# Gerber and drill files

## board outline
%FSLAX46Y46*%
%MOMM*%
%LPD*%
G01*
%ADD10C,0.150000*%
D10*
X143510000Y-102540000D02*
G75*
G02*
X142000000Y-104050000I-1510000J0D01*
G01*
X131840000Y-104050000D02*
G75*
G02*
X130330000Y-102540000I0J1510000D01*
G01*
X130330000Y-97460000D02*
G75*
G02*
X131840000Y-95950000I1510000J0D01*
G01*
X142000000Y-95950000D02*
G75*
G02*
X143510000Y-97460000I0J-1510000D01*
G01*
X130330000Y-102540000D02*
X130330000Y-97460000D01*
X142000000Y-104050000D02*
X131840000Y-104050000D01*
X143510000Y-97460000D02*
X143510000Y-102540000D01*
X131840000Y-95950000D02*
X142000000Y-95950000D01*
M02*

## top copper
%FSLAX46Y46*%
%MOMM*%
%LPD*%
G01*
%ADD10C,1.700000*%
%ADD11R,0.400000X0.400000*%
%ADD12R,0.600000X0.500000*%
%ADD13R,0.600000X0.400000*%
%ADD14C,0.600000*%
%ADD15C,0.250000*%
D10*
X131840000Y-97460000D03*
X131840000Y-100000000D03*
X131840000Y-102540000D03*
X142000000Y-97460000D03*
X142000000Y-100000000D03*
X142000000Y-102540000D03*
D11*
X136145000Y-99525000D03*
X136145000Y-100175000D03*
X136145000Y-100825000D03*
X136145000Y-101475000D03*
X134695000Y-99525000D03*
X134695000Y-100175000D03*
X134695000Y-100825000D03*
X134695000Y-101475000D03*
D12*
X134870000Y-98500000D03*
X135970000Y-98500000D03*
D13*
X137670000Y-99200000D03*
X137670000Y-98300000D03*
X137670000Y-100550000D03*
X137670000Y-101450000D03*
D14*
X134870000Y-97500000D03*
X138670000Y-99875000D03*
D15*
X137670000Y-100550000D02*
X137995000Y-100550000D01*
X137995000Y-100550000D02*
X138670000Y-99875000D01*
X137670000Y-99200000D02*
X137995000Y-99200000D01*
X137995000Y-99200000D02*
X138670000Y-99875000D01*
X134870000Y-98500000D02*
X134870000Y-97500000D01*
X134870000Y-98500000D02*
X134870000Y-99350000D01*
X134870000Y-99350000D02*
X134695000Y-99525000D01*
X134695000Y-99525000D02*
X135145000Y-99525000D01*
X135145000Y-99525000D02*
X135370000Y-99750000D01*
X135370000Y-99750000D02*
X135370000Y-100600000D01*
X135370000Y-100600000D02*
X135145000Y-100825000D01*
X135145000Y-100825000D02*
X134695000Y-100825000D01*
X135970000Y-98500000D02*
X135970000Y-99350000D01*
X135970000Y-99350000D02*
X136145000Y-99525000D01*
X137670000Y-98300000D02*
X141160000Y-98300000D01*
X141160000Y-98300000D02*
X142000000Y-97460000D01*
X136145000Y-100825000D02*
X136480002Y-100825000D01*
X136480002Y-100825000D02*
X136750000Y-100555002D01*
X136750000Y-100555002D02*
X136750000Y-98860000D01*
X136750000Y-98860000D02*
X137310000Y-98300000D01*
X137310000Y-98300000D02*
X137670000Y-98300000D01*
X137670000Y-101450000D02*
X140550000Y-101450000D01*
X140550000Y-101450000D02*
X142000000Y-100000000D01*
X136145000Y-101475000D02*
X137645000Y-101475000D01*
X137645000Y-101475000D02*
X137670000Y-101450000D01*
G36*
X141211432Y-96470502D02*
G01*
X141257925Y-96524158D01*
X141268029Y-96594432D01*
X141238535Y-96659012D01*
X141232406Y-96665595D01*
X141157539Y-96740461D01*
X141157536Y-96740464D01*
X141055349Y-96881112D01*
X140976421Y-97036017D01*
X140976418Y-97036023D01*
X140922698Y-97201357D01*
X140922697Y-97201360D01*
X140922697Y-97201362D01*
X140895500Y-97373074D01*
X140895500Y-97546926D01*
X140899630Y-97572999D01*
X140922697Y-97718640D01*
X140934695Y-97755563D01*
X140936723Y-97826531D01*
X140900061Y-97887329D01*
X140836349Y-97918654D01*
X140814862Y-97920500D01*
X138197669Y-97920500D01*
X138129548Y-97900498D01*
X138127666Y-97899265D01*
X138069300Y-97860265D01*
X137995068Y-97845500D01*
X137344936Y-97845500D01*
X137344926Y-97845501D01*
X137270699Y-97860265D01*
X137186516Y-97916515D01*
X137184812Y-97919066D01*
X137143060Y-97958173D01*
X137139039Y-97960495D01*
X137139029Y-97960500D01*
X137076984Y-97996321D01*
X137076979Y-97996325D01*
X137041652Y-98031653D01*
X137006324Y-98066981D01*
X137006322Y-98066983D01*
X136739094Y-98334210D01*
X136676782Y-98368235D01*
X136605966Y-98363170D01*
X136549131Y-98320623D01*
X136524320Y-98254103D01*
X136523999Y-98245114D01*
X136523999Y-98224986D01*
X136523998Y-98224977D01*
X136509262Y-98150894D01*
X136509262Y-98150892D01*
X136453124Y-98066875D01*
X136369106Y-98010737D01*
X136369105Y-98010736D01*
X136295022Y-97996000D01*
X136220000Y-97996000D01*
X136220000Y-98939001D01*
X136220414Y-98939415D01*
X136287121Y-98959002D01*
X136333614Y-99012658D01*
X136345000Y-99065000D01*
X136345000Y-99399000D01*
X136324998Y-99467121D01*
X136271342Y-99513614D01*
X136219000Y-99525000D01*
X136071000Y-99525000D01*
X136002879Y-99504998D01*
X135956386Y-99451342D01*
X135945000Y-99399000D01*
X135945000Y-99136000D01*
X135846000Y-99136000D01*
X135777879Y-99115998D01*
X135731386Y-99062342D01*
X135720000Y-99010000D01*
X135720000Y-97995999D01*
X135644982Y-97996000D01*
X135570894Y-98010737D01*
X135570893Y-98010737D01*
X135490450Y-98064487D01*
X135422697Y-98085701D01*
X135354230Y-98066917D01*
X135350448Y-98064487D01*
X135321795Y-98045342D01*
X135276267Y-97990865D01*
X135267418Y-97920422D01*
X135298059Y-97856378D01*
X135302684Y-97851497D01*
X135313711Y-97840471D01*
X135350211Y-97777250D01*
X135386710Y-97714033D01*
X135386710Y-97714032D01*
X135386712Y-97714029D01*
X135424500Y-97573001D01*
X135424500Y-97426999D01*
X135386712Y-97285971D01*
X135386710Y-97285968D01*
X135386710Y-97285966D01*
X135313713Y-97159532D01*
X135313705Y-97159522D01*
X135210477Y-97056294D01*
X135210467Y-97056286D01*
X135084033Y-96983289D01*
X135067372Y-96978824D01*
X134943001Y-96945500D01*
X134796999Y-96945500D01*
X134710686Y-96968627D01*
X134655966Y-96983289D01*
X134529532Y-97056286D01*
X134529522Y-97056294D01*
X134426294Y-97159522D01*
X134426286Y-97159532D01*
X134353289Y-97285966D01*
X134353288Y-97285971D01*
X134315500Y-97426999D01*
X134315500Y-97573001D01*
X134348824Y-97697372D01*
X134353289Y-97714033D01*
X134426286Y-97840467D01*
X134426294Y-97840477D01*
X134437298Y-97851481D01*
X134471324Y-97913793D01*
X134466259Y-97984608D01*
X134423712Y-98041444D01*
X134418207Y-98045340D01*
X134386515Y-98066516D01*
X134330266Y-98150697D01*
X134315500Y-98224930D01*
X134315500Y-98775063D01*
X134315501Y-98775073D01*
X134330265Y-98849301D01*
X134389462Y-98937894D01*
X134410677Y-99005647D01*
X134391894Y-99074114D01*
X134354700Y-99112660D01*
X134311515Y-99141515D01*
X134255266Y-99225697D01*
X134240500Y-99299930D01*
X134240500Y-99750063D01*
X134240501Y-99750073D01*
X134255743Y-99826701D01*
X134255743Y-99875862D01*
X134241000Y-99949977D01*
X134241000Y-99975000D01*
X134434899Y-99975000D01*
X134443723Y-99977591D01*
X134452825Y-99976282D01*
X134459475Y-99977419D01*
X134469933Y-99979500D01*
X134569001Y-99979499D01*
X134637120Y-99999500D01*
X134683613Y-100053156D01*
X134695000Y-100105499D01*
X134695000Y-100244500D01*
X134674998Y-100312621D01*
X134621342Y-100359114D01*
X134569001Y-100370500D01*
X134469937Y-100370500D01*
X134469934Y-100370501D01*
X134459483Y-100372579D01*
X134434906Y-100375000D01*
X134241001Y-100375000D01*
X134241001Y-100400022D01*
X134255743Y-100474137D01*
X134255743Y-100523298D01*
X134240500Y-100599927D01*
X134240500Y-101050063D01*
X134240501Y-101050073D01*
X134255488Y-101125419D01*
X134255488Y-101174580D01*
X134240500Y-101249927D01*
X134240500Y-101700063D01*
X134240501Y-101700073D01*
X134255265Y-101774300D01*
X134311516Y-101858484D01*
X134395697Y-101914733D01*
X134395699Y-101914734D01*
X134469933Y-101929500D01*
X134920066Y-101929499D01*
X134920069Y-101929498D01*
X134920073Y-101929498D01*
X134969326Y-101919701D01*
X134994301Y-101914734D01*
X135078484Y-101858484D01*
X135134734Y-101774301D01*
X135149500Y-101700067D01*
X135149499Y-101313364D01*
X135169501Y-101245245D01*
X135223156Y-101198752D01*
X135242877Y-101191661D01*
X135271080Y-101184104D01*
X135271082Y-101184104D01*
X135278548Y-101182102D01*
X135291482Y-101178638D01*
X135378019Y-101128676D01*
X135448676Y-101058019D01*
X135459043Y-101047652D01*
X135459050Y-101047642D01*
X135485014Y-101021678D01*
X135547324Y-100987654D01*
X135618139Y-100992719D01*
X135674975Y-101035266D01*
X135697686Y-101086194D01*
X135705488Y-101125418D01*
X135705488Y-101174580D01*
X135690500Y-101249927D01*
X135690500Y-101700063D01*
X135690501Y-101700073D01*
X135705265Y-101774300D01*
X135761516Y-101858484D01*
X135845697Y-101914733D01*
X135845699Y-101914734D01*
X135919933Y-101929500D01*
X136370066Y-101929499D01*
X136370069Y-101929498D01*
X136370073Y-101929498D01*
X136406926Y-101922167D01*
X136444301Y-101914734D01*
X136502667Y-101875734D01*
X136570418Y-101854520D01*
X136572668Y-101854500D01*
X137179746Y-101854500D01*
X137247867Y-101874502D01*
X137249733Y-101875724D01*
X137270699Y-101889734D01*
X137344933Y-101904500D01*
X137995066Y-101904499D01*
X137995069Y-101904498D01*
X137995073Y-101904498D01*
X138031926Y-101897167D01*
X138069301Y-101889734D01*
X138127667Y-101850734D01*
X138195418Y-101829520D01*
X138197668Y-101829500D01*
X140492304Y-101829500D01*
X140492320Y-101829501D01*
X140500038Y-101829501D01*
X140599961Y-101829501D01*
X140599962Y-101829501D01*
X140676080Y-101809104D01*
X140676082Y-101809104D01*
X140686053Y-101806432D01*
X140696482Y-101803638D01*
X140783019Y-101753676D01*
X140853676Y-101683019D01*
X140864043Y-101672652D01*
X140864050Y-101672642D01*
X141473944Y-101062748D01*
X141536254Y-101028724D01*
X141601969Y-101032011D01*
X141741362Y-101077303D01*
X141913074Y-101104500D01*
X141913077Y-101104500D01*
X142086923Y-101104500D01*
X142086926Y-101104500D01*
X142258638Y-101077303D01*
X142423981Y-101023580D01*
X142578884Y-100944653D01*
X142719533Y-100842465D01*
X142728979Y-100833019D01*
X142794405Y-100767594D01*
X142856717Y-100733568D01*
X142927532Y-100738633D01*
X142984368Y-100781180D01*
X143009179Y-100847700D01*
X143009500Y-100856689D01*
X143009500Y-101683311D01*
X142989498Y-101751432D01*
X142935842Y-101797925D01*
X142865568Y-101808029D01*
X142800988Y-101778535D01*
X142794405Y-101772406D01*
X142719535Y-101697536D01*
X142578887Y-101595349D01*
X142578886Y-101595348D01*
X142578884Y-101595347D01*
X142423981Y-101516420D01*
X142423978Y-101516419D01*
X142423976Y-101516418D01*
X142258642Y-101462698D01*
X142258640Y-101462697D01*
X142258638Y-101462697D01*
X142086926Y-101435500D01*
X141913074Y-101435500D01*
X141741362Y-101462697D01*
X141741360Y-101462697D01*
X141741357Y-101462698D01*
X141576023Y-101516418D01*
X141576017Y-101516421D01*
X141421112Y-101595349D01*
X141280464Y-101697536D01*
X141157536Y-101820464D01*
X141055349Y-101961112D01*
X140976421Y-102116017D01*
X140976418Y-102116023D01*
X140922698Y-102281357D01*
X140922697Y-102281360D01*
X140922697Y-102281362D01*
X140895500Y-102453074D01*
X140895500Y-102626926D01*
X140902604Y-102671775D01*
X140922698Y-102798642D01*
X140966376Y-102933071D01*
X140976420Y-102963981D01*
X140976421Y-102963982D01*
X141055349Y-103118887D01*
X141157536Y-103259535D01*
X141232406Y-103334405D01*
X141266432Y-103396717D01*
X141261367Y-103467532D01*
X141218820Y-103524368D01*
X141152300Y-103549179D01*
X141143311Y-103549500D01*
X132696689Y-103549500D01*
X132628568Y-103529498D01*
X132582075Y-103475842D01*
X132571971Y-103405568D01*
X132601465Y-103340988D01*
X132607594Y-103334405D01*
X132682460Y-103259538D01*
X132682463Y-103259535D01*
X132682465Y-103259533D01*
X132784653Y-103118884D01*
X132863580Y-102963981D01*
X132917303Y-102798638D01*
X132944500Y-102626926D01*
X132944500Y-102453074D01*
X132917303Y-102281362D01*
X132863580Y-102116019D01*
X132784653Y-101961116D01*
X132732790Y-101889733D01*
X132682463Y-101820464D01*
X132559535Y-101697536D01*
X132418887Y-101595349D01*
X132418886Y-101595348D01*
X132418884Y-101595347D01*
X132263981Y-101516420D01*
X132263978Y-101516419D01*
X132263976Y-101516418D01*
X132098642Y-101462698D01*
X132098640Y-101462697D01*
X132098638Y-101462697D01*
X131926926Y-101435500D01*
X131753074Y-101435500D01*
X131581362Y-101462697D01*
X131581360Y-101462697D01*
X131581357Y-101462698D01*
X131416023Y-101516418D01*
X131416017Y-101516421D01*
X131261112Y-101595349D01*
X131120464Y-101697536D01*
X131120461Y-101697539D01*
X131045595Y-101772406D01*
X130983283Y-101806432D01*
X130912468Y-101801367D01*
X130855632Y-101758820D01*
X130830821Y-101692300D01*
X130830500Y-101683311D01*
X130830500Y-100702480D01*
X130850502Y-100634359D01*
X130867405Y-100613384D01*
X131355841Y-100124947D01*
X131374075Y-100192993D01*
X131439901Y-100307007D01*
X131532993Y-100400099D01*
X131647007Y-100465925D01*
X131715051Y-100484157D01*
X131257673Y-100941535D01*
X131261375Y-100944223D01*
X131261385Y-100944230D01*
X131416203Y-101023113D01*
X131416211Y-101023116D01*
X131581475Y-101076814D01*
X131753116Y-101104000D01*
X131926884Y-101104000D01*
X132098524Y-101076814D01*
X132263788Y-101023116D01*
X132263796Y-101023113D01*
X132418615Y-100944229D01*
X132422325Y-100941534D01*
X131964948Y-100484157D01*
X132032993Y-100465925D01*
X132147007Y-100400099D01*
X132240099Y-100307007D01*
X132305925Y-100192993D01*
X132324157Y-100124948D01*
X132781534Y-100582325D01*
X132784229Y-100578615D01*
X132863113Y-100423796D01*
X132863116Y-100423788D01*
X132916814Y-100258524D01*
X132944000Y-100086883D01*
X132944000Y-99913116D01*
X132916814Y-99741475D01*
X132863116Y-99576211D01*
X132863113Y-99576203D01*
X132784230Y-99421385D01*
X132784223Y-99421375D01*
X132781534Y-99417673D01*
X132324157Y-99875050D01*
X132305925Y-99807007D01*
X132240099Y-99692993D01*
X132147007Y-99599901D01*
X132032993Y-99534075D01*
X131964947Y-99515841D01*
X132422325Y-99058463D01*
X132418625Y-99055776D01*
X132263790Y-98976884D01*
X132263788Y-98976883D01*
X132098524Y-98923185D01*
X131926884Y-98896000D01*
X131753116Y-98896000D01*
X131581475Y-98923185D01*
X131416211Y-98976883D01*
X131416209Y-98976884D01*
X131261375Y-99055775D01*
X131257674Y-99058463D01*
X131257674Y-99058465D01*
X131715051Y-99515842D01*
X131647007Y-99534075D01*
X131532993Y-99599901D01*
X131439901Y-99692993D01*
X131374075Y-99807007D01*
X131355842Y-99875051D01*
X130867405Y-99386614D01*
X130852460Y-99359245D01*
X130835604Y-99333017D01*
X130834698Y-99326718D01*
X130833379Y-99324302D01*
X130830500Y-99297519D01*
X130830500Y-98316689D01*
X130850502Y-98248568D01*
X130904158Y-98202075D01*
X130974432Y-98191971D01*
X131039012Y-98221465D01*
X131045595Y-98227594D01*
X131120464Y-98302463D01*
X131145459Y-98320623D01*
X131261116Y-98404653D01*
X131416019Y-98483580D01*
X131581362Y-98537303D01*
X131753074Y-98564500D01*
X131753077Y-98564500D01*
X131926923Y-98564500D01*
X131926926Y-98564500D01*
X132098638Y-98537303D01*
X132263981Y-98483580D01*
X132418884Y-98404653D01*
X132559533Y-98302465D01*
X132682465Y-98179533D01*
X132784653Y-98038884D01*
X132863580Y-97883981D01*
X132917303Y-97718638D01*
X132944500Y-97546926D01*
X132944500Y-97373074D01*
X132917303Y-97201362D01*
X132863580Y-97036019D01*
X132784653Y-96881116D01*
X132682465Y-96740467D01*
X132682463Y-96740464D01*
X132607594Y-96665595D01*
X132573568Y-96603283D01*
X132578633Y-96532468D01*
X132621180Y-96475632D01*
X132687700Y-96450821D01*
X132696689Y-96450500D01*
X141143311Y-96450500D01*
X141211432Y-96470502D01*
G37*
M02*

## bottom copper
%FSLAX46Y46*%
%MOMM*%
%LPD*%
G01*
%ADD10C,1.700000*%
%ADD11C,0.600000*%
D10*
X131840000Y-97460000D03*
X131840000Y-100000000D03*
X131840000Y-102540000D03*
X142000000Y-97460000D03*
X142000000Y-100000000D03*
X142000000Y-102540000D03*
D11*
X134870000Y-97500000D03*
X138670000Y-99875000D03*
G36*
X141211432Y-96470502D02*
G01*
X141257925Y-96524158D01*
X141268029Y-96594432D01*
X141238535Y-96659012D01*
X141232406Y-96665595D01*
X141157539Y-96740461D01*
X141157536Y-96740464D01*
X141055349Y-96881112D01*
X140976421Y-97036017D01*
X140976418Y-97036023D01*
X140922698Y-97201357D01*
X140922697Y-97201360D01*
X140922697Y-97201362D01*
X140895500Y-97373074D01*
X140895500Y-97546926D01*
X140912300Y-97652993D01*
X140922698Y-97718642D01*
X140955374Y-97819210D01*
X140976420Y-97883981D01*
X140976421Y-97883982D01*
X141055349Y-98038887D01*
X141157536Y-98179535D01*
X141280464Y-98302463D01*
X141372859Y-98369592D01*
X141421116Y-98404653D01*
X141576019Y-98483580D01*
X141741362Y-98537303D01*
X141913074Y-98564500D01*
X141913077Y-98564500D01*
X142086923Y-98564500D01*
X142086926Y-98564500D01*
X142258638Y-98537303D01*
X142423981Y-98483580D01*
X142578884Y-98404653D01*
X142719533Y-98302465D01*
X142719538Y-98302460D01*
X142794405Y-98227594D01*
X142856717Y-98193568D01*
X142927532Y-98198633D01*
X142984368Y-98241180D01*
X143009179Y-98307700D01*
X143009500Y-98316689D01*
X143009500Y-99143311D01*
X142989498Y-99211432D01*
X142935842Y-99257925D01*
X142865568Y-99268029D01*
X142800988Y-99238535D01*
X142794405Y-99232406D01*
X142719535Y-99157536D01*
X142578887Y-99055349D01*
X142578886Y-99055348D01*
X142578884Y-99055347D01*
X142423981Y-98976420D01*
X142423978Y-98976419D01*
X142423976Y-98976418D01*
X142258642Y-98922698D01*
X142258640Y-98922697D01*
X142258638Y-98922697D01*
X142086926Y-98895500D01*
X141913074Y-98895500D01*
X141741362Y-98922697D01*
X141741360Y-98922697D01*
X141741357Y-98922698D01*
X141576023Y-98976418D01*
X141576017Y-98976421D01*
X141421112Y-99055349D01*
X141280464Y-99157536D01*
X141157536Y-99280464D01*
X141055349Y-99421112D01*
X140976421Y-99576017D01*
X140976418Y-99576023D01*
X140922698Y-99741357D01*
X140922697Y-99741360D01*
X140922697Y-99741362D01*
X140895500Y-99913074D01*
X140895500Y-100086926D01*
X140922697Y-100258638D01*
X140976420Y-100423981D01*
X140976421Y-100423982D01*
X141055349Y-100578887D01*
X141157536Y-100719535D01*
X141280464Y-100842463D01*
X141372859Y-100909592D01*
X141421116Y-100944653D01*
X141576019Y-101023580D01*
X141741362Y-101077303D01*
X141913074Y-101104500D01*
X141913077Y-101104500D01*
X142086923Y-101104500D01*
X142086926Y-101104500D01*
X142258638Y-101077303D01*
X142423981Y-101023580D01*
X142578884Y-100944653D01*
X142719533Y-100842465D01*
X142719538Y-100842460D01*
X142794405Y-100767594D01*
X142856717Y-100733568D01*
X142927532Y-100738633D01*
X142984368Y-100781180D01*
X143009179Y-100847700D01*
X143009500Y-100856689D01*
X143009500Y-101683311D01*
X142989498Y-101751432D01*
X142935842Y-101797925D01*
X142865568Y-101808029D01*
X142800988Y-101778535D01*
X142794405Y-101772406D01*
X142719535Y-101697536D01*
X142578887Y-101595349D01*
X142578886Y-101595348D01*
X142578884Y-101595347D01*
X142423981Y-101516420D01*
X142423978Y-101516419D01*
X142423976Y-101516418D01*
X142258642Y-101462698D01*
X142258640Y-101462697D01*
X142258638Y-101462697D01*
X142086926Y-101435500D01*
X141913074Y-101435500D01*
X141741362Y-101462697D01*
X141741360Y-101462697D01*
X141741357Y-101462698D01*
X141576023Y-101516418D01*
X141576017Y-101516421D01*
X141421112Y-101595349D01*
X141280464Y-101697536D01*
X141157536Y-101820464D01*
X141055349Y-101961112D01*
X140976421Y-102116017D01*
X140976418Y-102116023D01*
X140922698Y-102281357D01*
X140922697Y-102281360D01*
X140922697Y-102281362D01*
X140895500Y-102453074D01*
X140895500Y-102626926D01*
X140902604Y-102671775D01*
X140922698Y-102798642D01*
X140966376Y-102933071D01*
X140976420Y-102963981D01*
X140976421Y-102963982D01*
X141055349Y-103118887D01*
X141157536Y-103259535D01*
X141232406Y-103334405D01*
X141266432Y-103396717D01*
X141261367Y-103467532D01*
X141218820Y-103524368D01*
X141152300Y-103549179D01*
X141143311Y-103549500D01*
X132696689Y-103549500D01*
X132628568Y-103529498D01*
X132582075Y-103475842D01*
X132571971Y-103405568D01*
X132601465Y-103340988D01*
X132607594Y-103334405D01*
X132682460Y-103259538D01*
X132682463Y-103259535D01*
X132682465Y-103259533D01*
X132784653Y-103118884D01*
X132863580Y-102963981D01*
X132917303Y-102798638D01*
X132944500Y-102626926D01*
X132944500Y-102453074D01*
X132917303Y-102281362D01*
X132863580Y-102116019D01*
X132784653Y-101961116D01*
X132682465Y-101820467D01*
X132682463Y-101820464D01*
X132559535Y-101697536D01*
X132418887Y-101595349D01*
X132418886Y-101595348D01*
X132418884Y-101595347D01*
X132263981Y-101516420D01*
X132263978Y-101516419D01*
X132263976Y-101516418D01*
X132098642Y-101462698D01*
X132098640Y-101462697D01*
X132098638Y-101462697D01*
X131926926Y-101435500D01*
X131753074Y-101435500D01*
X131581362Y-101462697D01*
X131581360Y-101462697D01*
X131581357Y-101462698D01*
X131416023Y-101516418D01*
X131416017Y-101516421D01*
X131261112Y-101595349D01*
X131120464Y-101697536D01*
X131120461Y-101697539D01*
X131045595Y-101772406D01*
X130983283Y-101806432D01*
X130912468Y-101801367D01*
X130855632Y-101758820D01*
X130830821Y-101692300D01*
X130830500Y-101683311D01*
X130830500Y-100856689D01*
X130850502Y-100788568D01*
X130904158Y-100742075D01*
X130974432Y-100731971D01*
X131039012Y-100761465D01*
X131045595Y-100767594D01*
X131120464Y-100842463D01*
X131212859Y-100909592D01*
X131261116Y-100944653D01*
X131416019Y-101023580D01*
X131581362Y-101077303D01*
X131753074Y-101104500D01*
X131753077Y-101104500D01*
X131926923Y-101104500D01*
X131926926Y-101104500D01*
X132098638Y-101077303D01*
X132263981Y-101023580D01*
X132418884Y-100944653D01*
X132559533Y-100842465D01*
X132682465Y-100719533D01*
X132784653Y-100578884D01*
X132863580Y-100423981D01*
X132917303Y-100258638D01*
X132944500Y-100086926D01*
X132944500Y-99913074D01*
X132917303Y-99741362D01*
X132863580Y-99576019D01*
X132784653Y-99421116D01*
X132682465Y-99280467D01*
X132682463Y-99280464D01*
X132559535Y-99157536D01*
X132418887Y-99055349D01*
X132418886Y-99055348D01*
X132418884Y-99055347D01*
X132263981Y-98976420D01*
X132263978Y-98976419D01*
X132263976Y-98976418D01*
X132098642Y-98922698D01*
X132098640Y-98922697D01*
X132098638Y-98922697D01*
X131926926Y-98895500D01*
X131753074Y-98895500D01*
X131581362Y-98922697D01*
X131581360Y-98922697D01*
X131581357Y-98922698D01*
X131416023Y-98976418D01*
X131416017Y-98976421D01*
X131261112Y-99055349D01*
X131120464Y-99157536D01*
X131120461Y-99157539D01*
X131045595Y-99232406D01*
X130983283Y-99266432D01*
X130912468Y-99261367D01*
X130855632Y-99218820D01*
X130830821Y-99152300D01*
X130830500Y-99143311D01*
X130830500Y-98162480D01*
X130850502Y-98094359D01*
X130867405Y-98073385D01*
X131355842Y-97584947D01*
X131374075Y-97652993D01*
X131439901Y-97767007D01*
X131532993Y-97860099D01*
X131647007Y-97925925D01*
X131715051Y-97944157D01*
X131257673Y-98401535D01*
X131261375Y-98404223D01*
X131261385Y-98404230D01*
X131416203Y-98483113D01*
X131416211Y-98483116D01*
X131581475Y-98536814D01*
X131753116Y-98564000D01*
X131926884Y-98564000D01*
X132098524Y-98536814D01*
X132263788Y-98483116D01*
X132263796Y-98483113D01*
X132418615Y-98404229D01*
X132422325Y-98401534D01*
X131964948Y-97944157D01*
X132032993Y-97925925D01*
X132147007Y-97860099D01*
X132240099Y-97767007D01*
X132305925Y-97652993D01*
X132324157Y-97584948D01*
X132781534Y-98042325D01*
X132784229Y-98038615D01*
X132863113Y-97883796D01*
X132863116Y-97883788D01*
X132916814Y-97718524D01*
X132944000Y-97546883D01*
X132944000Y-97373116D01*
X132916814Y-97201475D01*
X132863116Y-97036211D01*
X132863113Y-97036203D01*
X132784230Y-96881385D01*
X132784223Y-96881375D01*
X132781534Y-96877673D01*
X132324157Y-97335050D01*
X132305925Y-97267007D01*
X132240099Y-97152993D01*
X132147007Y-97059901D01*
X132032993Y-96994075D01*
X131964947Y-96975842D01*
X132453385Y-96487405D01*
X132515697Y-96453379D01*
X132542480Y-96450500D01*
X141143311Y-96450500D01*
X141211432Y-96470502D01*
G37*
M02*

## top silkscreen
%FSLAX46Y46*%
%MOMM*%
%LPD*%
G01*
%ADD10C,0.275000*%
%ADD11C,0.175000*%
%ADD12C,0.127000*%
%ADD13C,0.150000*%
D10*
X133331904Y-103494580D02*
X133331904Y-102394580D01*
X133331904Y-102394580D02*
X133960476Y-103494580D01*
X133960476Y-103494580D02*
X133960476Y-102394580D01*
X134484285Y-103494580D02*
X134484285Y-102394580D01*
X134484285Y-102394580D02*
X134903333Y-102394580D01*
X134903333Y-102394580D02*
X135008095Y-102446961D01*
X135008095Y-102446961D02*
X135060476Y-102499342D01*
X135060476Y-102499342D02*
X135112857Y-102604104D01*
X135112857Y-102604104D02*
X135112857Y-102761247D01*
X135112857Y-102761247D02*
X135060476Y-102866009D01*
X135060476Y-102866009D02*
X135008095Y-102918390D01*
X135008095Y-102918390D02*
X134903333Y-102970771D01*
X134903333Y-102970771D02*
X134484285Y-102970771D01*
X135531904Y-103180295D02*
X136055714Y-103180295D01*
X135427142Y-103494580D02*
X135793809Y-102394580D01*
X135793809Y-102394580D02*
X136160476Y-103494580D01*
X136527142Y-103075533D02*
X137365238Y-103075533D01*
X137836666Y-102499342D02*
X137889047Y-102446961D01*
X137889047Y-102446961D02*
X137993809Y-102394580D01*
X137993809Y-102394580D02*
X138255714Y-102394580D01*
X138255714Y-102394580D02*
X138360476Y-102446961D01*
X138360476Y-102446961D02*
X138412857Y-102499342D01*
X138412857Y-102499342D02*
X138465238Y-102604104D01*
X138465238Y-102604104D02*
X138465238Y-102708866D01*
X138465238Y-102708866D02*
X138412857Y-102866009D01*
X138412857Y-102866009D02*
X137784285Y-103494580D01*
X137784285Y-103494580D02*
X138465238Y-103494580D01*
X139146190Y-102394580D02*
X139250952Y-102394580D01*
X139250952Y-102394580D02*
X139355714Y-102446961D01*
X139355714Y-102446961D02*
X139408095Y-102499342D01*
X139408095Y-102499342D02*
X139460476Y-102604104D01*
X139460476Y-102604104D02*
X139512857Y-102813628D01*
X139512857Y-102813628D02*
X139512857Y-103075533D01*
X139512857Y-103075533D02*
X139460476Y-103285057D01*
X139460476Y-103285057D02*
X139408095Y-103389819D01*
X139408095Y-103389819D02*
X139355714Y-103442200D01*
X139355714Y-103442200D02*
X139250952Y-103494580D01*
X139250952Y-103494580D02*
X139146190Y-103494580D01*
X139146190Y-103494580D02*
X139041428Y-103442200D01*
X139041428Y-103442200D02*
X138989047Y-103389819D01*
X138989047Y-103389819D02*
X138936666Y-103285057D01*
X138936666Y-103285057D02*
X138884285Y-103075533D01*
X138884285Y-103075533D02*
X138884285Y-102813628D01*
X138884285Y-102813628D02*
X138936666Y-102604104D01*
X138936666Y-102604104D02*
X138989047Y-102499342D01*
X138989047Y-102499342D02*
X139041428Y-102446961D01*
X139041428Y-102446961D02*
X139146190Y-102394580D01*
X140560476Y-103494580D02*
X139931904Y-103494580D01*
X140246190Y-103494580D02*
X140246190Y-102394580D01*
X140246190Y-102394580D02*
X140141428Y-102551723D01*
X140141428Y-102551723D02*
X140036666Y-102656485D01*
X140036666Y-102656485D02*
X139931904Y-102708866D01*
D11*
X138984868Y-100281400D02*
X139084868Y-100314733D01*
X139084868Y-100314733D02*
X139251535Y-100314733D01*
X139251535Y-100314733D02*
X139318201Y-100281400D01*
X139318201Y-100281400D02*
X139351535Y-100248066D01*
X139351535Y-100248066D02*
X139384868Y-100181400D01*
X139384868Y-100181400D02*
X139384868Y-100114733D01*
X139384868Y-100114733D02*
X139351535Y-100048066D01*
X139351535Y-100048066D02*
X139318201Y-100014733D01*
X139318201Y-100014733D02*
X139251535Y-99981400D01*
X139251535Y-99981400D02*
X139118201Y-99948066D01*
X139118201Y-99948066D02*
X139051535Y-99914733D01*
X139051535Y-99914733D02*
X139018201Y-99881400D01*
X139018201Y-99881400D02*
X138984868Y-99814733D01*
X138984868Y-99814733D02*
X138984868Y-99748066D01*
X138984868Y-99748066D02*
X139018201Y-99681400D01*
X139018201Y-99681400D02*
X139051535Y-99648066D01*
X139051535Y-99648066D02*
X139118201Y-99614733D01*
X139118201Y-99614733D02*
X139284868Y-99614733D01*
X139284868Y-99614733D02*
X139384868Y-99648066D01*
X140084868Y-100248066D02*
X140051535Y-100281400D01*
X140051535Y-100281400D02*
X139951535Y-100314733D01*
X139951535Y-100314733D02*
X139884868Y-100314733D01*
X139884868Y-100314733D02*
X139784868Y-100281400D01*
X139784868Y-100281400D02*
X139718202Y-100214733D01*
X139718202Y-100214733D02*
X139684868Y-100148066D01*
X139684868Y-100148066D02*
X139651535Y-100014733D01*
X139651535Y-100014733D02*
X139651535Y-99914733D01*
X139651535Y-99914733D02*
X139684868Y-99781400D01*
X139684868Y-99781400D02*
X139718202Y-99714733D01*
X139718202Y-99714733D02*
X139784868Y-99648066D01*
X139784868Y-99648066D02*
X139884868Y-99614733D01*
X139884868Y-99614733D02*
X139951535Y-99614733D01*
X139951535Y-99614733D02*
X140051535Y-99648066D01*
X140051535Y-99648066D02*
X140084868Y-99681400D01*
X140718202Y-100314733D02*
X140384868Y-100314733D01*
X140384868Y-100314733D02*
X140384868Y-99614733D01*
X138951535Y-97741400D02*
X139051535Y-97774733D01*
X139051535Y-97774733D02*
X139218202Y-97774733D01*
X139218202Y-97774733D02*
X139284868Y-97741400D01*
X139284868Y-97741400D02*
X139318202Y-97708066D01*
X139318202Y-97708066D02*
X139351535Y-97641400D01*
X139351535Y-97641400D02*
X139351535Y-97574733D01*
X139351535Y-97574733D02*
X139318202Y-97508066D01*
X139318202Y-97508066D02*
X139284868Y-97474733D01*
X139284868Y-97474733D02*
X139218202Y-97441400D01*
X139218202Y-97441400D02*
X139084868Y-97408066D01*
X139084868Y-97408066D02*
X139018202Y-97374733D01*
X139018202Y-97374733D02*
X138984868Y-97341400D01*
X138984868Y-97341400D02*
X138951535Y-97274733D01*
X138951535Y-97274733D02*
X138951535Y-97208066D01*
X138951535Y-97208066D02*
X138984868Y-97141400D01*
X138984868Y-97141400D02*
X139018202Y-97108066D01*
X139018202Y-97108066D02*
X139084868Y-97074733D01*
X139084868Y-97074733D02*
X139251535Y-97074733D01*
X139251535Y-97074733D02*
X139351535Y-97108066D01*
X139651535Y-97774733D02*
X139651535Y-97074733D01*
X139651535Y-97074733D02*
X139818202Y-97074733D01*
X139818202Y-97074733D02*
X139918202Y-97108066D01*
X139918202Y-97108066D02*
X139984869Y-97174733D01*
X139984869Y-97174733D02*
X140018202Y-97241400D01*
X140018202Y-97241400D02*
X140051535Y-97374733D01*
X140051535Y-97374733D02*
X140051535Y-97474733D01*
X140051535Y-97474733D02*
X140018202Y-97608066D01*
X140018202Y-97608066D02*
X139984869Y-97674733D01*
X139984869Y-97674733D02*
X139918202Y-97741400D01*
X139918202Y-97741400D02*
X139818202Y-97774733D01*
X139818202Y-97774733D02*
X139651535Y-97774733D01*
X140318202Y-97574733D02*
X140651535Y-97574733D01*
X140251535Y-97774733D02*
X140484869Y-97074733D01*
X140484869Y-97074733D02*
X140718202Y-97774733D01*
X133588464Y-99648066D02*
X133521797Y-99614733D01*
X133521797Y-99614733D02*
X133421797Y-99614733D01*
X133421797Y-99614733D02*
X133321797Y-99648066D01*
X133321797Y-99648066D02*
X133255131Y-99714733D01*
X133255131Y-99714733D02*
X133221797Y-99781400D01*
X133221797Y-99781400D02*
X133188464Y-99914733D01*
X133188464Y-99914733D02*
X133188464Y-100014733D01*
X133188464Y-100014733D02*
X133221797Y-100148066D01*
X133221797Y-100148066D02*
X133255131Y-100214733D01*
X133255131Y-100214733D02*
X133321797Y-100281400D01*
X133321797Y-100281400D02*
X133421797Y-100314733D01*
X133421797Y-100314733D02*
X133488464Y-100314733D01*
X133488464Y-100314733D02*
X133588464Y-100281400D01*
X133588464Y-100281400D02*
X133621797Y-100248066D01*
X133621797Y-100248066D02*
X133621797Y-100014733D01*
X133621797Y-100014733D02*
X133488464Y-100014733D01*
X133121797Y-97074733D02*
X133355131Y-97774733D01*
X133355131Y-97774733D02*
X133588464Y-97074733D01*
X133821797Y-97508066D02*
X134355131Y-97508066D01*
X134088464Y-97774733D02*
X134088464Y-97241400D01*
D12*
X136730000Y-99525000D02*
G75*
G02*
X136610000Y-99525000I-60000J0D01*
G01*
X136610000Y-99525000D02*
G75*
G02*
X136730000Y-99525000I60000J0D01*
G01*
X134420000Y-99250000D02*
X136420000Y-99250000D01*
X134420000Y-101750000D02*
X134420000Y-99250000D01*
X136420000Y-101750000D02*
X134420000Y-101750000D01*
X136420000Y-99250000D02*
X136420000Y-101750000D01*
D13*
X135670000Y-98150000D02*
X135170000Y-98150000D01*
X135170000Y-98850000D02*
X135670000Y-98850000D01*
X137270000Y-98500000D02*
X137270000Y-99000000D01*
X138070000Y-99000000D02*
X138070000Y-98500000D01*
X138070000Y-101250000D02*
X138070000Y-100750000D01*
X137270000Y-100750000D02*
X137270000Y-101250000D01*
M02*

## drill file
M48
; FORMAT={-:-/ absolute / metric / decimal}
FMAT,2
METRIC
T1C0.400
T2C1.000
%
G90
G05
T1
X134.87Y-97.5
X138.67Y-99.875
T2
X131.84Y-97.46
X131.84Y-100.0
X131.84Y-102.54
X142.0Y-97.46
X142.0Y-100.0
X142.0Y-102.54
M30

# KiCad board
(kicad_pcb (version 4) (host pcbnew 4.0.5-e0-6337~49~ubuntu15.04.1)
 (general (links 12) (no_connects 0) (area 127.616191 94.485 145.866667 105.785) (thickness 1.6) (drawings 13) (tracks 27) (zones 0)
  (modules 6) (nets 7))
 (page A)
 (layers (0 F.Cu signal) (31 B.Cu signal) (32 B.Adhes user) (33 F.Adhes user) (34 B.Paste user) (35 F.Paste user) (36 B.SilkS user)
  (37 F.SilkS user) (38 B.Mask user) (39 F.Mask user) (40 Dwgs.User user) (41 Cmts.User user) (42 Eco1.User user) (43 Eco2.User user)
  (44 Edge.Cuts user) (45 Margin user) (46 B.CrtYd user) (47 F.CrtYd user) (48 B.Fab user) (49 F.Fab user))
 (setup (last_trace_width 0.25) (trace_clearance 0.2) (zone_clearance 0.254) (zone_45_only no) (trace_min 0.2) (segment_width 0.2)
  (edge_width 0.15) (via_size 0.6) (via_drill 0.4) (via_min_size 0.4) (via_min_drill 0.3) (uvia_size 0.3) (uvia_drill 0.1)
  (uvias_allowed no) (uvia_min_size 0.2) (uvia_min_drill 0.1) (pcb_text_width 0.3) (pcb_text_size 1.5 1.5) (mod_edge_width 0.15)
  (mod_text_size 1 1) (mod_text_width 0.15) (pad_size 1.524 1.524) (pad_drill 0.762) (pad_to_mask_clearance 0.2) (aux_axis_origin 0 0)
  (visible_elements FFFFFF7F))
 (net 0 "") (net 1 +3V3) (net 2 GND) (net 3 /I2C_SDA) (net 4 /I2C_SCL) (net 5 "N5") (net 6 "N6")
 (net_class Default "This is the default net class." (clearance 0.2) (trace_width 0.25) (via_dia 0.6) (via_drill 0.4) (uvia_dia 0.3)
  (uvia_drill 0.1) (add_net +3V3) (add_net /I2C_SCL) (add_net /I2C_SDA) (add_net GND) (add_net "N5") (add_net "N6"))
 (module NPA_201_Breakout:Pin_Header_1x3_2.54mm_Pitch (layer F.Cu) (at 131.84 97.46)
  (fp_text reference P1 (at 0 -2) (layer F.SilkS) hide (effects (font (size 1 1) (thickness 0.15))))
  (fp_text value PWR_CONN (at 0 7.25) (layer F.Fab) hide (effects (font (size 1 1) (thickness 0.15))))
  (pad 1 thru_hole circle (at 0 0) (size 1.7 1.7) (drill 1) (layers *.Cu *.Mask) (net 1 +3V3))
  (pad 2 thru_hole circle (at 0 2.54) (size 1.7 1.7) (drill 1) (layers *.Cu *.Mask) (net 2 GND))
  (pad 3 thru_hole circle (at 0 5.08) (size 1.7 1.7) (drill 1) (layers *.Cu *.Mask)))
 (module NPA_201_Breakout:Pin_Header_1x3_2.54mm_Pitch (layer F.Cu) (at 142 97.46)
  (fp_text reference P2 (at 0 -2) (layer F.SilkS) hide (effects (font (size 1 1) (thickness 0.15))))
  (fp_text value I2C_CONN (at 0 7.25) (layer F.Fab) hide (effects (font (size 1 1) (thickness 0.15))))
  (pad 1 thru_hole circle (at 0 0) (size 1.7 1.7) (drill 1) (layers *.Cu *.Mask) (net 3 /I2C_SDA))
  (pad 2 thru_hole circle (at 0 2.54) (size 1.7 1.7) (drill 1) (layers *.Cu *.Mask) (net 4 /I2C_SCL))
  (pad 3 thru_hole circle (at 0 5.08) (size 1.7 1.7) (drill 1) (layers *.Cu *.Mask)))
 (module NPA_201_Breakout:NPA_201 (layer F.Cu) (at 135.42 100.5 270)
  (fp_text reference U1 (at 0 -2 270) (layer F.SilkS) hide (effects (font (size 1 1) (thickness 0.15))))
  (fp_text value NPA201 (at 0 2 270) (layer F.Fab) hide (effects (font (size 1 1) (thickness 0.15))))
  (fp_circle (center -0.975 -1.25) (end -0.975 -1.19) (layer F.SilkS) (width 0.127))
  (fp_line (start -1.25 1) (end -1.25 -1) (layer F.SilkS) (width 0.127))
  (fp_line (start 1.25 1) (end -1.25 1) (layer F.SilkS) (width 0.127))
  (fp_line (start 1.25 -1) (end 1.25 1) (layer F.SilkS) (width 0.127))
  (fp_line (start -1.25 -1) (end 1.25 -1) (layer F.SilkS) (width 0.127))
  (pad 1 smd rect (at -0.975 -0.725 270) (size 0.4 0.4) (layers F.Cu F.Paste F.Mask) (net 2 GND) (solder_mask_margin 0.05)
   (solder_paste_margin -0.025))
  (pad 2 smd rect (at -0.325 -0.725 270) (size 0.4 0.4) (layers F.Cu F.Paste F.Mask) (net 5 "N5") (solder_mask_margin 0.05)
   (solder_paste_margin -0.025))
  (pad 3 smd rect (at 0.325 -0.725 270) (size 0.4 0.4) (layers F.Cu F.Paste F.Mask) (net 3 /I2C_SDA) (solder_mask_margin 0.05)
   (solder_paste_margin -0.025))
  (pad 4 smd rect (at 0.975 -0.725 270) (size 0.4 0.4) (layers F.Cu F.Paste F.Mask) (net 4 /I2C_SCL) (solder_mask_margin 0.05)
   (solder_paste_margin -0.025))
  (pad 8 smd rect (at -0.975 0.725 270) (size 0.4 0.4) (layers F.Cu F.Paste F.Mask) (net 1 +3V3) (solder_mask_margin 0.05)
   (solder_paste_margin -0.025))
  (pad 7 smd rect (at -0.325 0.725 270) (size 0.4 0.4) (layers F.Cu F.Paste F.Mask) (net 2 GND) (solder_mask_margin 0.05)
   (solder_paste_margin -0.025))
  (pad 6 smd rect (at 0.325 0.725 270) (size 0.4 0.4) (layers F.Cu F.Paste F.Mask) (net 1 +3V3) (solder_mask_margin 0.05)
   (solder_paste_margin -0.025))
  (pad 5 smd rect (at 0.975 0.725 270) (size 0.4 0.4) (layers F.Cu F.Paste F.Mask) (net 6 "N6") (solder_mask_margin 0.05)
   (solder_paste_margin -0.025)))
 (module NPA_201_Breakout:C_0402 (layer F.Cu) (at 135.42 98.5)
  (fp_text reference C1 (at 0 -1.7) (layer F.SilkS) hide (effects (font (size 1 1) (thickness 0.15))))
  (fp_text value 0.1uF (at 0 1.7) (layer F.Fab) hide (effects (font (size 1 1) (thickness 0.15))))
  (fp_line (start 0.25 -0.35) (end -0.25 -0.35) (layer F.SilkS) (width 0.15))
  (fp_line (start -0.25 0.35) (end 0.25 0.35) (layer F.SilkS) (width 0.15))
  (pad 1 smd rect (at -0.55 0) (size 0.6 0.5) (layers F.Cu F.Paste F.Mask) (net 1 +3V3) (solder_mask_margin 0.1))
  (pad 2 smd rect (at 0.55 0) (size 0.6 0.5) (layers F.Cu F.Paste F.Mask) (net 2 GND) (solder_mask_margin 0.1)))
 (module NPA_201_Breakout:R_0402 (layer F.Cu) (at 137.67 98.75 90)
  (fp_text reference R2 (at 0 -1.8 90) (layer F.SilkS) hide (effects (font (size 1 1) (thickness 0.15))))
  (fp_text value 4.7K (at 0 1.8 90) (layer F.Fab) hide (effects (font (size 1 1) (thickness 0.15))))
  (fp_line (start 0.25 -0.4) (end -0.25 -0.4) (layer F.SilkS) (width 0.15))
  (fp_line (start -0.25 0.4) (end 0.25 0.4) (layer F.SilkS) (width 0.15))
  (pad 1 smd rect (at -0.45 0 90) (size 0.4 0.6) (layers F.Cu F.Paste F.Mask) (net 1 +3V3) (solder_mask_margin 0.1))
  (pad 2 smd rect (at 0.45 0 90) (size 0.4 0.6) (layers F.Cu F.Paste F.Mask) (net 3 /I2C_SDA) (solder_mask_margin 0.1)))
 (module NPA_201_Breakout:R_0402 (layer F.Cu) (at 137.67 101 270)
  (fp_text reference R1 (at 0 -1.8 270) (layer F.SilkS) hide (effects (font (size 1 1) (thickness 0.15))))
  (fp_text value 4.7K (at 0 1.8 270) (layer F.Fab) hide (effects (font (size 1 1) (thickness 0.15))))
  (fp_line (start 0.25 -0.4) (end -0.25 -0.4) (layer F.SilkS) (width 0.15))
  (fp_line (start -0.25 0.4) (end 0.25 0.4) (layer F.SilkS) (width 0.15))
  (pad 1 smd rect (at -0.45 0 270) (size 0.4 0.6) (layers F.Cu F.Paste F.Mask) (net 1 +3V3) (solder_mask_margin 0.1))
  (pad 2 smd rect (at 0.45 0 270) (size 0.4 0.6) (layers F.Cu F.Paste F.Mask) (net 4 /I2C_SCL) (solder_mask_margin 0.1)))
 (gr_arc (start 142 102.54) (end 143.51 102.54) (angle 90) (layer Edge.Cuts) (width 0.15))
 (gr_arc (start 131.84 102.54) (end 131.84 104.05) (angle 90) (layer Edge.Cuts) (width 0.15))
 (gr_arc (start 131.84 97.46) (end 130.33 97.46) (angle 90) (layer Edge.Cuts) (width 0.15))
 (gr_arc (start 142 97.46) (end 142 95.95) (angle 90) (layer Edge.Cuts) (width 0.15))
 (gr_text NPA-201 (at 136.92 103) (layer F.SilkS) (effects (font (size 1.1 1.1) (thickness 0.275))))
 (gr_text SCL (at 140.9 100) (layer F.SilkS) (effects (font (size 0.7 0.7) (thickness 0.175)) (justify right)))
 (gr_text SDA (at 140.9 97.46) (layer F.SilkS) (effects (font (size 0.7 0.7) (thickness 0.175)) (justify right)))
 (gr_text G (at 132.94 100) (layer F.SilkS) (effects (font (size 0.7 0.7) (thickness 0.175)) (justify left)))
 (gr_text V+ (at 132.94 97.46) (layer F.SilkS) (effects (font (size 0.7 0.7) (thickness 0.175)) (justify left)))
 (gr_line (start 130.33 102.54) (end 130.33 97.46) (layer Edge.Cuts) (width 0.15))
 (gr_line (start 142 104.05) (end 131.84 104.05) (layer Edge.Cuts) (width 0.15))
 (gr_line (start 143.51 97.46) (end 143.51 102.54) (layer Edge.Cuts) (width 0.15))
 (gr_line (start 131.84 95.95) (end 142 95.95) (layer Edge.Cuts) (width 0.15))
 (segment (start 137.67 100.55) (end 137.995 100.55) (width 0.25) (layer F.Cu) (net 1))
 (segment (start 137.995 100.55) (end 138.67 99.875) (width 0.25) (layer F.Cu) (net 1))
 (segment (start 137.67 99.2) (end 137.995 99.2) (width 0.25) (layer F.Cu) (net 1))
 (segment (start 137.995 99.2) (end 138.67 99.875) (width 0.25) (layer F.Cu) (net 1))
 (segment (start 134.87 98.5) (end 134.87 97.5) (width 0.25) (layer F.Cu) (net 1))
 (via (at 134.87 97.5) (size 0.6) (drill 0.4) (layers F.Cu B.Cu) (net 1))
 (via (at 138.67 99.875) (size 0.6) (drill 0.4) (layers F.Cu B.Cu) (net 1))
 (segment (start 134.87 98.5) (end 134.87 99.35) (width 0.25) (layer F.Cu) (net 1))
 (segment (start 134.87 99.35) (end 134.695 99.525) (width 0.25) (layer F.Cu) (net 1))
 (segment (start 134.695 99.525) (end 135.145 99.525) (width 0.25) (layer F.Cu) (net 1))
 (segment (start 135.145 99.525) (end 135.37 99.75) (width 0.25) (layer F.Cu) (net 1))
 (segment (start 135.37 99.75) (end 135.37 100.6) (width 0.25) (layer F.Cu) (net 1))
 (segment (start 135.37 100.6) (end 135.145 100.825) (width 0.25) (layer F.Cu) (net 1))
 (segment (start 135.145 100.825) (end 134.695 100.825) (width 0.25) (layer F.Cu) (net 1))
 (segment (start 135.97 98.5) (end 135.97 99.35) (width 0.25) (layer F.Cu) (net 2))
 (segment (start 135.97 99.35) (end 136.145 99.525) (width 0.25) (layer F.Cu) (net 2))
 (segment (start 137.67 98.3) (end 141.16 98.3) (width 0.25) (layer F.Cu) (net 3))
 (segment (start 141.16 98.3) (end 142 97.46) (width 0.25) (layer F.Cu) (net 3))
 (segment (start 136.145 100.825) (end 136.480002 100.825) (width 0.25) (layer F.Cu) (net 3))
 (segment (start 136.480002 100.825) (end 136.75 100.555002) (width 0.25) (layer F.Cu) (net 3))
 (segment (start 136.75 100.555002) (end 136.75 98.86) (width 0.25) (layer F.Cu) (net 3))
 (segment (start 136.75 98.86) (end 137.31 98.3) (width 0.25) (layer F.Cu) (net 3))
 (segment (start 137.31 98.3) (end 137.67 98.3) (width 0.25) (layer F.Cu) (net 3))
 (segment (start 137.67 101.45) (end 140.55 101.45) (width 0.25) (layer F.Cu) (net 4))
 (segment (start 140.55 101.45) (end 142 100) (width 0.25) (layer F.Cu) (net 4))
 (segment (start 136.145 101.475) (end 137.645 101.475) (width 0.25) (layer F.Cu) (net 4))
 (segment (start 137.645 101.475) (end 137.67 101.45) (width 0.25) (layer F.Cu) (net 4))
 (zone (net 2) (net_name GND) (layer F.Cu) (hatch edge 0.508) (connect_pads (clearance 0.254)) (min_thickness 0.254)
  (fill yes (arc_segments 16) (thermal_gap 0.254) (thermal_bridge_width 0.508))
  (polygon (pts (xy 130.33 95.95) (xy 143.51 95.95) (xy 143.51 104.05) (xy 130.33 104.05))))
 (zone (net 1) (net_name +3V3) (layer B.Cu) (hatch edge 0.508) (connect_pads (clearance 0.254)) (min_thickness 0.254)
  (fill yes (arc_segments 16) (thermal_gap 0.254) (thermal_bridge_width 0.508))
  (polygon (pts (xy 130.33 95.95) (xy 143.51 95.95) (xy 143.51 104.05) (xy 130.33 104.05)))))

